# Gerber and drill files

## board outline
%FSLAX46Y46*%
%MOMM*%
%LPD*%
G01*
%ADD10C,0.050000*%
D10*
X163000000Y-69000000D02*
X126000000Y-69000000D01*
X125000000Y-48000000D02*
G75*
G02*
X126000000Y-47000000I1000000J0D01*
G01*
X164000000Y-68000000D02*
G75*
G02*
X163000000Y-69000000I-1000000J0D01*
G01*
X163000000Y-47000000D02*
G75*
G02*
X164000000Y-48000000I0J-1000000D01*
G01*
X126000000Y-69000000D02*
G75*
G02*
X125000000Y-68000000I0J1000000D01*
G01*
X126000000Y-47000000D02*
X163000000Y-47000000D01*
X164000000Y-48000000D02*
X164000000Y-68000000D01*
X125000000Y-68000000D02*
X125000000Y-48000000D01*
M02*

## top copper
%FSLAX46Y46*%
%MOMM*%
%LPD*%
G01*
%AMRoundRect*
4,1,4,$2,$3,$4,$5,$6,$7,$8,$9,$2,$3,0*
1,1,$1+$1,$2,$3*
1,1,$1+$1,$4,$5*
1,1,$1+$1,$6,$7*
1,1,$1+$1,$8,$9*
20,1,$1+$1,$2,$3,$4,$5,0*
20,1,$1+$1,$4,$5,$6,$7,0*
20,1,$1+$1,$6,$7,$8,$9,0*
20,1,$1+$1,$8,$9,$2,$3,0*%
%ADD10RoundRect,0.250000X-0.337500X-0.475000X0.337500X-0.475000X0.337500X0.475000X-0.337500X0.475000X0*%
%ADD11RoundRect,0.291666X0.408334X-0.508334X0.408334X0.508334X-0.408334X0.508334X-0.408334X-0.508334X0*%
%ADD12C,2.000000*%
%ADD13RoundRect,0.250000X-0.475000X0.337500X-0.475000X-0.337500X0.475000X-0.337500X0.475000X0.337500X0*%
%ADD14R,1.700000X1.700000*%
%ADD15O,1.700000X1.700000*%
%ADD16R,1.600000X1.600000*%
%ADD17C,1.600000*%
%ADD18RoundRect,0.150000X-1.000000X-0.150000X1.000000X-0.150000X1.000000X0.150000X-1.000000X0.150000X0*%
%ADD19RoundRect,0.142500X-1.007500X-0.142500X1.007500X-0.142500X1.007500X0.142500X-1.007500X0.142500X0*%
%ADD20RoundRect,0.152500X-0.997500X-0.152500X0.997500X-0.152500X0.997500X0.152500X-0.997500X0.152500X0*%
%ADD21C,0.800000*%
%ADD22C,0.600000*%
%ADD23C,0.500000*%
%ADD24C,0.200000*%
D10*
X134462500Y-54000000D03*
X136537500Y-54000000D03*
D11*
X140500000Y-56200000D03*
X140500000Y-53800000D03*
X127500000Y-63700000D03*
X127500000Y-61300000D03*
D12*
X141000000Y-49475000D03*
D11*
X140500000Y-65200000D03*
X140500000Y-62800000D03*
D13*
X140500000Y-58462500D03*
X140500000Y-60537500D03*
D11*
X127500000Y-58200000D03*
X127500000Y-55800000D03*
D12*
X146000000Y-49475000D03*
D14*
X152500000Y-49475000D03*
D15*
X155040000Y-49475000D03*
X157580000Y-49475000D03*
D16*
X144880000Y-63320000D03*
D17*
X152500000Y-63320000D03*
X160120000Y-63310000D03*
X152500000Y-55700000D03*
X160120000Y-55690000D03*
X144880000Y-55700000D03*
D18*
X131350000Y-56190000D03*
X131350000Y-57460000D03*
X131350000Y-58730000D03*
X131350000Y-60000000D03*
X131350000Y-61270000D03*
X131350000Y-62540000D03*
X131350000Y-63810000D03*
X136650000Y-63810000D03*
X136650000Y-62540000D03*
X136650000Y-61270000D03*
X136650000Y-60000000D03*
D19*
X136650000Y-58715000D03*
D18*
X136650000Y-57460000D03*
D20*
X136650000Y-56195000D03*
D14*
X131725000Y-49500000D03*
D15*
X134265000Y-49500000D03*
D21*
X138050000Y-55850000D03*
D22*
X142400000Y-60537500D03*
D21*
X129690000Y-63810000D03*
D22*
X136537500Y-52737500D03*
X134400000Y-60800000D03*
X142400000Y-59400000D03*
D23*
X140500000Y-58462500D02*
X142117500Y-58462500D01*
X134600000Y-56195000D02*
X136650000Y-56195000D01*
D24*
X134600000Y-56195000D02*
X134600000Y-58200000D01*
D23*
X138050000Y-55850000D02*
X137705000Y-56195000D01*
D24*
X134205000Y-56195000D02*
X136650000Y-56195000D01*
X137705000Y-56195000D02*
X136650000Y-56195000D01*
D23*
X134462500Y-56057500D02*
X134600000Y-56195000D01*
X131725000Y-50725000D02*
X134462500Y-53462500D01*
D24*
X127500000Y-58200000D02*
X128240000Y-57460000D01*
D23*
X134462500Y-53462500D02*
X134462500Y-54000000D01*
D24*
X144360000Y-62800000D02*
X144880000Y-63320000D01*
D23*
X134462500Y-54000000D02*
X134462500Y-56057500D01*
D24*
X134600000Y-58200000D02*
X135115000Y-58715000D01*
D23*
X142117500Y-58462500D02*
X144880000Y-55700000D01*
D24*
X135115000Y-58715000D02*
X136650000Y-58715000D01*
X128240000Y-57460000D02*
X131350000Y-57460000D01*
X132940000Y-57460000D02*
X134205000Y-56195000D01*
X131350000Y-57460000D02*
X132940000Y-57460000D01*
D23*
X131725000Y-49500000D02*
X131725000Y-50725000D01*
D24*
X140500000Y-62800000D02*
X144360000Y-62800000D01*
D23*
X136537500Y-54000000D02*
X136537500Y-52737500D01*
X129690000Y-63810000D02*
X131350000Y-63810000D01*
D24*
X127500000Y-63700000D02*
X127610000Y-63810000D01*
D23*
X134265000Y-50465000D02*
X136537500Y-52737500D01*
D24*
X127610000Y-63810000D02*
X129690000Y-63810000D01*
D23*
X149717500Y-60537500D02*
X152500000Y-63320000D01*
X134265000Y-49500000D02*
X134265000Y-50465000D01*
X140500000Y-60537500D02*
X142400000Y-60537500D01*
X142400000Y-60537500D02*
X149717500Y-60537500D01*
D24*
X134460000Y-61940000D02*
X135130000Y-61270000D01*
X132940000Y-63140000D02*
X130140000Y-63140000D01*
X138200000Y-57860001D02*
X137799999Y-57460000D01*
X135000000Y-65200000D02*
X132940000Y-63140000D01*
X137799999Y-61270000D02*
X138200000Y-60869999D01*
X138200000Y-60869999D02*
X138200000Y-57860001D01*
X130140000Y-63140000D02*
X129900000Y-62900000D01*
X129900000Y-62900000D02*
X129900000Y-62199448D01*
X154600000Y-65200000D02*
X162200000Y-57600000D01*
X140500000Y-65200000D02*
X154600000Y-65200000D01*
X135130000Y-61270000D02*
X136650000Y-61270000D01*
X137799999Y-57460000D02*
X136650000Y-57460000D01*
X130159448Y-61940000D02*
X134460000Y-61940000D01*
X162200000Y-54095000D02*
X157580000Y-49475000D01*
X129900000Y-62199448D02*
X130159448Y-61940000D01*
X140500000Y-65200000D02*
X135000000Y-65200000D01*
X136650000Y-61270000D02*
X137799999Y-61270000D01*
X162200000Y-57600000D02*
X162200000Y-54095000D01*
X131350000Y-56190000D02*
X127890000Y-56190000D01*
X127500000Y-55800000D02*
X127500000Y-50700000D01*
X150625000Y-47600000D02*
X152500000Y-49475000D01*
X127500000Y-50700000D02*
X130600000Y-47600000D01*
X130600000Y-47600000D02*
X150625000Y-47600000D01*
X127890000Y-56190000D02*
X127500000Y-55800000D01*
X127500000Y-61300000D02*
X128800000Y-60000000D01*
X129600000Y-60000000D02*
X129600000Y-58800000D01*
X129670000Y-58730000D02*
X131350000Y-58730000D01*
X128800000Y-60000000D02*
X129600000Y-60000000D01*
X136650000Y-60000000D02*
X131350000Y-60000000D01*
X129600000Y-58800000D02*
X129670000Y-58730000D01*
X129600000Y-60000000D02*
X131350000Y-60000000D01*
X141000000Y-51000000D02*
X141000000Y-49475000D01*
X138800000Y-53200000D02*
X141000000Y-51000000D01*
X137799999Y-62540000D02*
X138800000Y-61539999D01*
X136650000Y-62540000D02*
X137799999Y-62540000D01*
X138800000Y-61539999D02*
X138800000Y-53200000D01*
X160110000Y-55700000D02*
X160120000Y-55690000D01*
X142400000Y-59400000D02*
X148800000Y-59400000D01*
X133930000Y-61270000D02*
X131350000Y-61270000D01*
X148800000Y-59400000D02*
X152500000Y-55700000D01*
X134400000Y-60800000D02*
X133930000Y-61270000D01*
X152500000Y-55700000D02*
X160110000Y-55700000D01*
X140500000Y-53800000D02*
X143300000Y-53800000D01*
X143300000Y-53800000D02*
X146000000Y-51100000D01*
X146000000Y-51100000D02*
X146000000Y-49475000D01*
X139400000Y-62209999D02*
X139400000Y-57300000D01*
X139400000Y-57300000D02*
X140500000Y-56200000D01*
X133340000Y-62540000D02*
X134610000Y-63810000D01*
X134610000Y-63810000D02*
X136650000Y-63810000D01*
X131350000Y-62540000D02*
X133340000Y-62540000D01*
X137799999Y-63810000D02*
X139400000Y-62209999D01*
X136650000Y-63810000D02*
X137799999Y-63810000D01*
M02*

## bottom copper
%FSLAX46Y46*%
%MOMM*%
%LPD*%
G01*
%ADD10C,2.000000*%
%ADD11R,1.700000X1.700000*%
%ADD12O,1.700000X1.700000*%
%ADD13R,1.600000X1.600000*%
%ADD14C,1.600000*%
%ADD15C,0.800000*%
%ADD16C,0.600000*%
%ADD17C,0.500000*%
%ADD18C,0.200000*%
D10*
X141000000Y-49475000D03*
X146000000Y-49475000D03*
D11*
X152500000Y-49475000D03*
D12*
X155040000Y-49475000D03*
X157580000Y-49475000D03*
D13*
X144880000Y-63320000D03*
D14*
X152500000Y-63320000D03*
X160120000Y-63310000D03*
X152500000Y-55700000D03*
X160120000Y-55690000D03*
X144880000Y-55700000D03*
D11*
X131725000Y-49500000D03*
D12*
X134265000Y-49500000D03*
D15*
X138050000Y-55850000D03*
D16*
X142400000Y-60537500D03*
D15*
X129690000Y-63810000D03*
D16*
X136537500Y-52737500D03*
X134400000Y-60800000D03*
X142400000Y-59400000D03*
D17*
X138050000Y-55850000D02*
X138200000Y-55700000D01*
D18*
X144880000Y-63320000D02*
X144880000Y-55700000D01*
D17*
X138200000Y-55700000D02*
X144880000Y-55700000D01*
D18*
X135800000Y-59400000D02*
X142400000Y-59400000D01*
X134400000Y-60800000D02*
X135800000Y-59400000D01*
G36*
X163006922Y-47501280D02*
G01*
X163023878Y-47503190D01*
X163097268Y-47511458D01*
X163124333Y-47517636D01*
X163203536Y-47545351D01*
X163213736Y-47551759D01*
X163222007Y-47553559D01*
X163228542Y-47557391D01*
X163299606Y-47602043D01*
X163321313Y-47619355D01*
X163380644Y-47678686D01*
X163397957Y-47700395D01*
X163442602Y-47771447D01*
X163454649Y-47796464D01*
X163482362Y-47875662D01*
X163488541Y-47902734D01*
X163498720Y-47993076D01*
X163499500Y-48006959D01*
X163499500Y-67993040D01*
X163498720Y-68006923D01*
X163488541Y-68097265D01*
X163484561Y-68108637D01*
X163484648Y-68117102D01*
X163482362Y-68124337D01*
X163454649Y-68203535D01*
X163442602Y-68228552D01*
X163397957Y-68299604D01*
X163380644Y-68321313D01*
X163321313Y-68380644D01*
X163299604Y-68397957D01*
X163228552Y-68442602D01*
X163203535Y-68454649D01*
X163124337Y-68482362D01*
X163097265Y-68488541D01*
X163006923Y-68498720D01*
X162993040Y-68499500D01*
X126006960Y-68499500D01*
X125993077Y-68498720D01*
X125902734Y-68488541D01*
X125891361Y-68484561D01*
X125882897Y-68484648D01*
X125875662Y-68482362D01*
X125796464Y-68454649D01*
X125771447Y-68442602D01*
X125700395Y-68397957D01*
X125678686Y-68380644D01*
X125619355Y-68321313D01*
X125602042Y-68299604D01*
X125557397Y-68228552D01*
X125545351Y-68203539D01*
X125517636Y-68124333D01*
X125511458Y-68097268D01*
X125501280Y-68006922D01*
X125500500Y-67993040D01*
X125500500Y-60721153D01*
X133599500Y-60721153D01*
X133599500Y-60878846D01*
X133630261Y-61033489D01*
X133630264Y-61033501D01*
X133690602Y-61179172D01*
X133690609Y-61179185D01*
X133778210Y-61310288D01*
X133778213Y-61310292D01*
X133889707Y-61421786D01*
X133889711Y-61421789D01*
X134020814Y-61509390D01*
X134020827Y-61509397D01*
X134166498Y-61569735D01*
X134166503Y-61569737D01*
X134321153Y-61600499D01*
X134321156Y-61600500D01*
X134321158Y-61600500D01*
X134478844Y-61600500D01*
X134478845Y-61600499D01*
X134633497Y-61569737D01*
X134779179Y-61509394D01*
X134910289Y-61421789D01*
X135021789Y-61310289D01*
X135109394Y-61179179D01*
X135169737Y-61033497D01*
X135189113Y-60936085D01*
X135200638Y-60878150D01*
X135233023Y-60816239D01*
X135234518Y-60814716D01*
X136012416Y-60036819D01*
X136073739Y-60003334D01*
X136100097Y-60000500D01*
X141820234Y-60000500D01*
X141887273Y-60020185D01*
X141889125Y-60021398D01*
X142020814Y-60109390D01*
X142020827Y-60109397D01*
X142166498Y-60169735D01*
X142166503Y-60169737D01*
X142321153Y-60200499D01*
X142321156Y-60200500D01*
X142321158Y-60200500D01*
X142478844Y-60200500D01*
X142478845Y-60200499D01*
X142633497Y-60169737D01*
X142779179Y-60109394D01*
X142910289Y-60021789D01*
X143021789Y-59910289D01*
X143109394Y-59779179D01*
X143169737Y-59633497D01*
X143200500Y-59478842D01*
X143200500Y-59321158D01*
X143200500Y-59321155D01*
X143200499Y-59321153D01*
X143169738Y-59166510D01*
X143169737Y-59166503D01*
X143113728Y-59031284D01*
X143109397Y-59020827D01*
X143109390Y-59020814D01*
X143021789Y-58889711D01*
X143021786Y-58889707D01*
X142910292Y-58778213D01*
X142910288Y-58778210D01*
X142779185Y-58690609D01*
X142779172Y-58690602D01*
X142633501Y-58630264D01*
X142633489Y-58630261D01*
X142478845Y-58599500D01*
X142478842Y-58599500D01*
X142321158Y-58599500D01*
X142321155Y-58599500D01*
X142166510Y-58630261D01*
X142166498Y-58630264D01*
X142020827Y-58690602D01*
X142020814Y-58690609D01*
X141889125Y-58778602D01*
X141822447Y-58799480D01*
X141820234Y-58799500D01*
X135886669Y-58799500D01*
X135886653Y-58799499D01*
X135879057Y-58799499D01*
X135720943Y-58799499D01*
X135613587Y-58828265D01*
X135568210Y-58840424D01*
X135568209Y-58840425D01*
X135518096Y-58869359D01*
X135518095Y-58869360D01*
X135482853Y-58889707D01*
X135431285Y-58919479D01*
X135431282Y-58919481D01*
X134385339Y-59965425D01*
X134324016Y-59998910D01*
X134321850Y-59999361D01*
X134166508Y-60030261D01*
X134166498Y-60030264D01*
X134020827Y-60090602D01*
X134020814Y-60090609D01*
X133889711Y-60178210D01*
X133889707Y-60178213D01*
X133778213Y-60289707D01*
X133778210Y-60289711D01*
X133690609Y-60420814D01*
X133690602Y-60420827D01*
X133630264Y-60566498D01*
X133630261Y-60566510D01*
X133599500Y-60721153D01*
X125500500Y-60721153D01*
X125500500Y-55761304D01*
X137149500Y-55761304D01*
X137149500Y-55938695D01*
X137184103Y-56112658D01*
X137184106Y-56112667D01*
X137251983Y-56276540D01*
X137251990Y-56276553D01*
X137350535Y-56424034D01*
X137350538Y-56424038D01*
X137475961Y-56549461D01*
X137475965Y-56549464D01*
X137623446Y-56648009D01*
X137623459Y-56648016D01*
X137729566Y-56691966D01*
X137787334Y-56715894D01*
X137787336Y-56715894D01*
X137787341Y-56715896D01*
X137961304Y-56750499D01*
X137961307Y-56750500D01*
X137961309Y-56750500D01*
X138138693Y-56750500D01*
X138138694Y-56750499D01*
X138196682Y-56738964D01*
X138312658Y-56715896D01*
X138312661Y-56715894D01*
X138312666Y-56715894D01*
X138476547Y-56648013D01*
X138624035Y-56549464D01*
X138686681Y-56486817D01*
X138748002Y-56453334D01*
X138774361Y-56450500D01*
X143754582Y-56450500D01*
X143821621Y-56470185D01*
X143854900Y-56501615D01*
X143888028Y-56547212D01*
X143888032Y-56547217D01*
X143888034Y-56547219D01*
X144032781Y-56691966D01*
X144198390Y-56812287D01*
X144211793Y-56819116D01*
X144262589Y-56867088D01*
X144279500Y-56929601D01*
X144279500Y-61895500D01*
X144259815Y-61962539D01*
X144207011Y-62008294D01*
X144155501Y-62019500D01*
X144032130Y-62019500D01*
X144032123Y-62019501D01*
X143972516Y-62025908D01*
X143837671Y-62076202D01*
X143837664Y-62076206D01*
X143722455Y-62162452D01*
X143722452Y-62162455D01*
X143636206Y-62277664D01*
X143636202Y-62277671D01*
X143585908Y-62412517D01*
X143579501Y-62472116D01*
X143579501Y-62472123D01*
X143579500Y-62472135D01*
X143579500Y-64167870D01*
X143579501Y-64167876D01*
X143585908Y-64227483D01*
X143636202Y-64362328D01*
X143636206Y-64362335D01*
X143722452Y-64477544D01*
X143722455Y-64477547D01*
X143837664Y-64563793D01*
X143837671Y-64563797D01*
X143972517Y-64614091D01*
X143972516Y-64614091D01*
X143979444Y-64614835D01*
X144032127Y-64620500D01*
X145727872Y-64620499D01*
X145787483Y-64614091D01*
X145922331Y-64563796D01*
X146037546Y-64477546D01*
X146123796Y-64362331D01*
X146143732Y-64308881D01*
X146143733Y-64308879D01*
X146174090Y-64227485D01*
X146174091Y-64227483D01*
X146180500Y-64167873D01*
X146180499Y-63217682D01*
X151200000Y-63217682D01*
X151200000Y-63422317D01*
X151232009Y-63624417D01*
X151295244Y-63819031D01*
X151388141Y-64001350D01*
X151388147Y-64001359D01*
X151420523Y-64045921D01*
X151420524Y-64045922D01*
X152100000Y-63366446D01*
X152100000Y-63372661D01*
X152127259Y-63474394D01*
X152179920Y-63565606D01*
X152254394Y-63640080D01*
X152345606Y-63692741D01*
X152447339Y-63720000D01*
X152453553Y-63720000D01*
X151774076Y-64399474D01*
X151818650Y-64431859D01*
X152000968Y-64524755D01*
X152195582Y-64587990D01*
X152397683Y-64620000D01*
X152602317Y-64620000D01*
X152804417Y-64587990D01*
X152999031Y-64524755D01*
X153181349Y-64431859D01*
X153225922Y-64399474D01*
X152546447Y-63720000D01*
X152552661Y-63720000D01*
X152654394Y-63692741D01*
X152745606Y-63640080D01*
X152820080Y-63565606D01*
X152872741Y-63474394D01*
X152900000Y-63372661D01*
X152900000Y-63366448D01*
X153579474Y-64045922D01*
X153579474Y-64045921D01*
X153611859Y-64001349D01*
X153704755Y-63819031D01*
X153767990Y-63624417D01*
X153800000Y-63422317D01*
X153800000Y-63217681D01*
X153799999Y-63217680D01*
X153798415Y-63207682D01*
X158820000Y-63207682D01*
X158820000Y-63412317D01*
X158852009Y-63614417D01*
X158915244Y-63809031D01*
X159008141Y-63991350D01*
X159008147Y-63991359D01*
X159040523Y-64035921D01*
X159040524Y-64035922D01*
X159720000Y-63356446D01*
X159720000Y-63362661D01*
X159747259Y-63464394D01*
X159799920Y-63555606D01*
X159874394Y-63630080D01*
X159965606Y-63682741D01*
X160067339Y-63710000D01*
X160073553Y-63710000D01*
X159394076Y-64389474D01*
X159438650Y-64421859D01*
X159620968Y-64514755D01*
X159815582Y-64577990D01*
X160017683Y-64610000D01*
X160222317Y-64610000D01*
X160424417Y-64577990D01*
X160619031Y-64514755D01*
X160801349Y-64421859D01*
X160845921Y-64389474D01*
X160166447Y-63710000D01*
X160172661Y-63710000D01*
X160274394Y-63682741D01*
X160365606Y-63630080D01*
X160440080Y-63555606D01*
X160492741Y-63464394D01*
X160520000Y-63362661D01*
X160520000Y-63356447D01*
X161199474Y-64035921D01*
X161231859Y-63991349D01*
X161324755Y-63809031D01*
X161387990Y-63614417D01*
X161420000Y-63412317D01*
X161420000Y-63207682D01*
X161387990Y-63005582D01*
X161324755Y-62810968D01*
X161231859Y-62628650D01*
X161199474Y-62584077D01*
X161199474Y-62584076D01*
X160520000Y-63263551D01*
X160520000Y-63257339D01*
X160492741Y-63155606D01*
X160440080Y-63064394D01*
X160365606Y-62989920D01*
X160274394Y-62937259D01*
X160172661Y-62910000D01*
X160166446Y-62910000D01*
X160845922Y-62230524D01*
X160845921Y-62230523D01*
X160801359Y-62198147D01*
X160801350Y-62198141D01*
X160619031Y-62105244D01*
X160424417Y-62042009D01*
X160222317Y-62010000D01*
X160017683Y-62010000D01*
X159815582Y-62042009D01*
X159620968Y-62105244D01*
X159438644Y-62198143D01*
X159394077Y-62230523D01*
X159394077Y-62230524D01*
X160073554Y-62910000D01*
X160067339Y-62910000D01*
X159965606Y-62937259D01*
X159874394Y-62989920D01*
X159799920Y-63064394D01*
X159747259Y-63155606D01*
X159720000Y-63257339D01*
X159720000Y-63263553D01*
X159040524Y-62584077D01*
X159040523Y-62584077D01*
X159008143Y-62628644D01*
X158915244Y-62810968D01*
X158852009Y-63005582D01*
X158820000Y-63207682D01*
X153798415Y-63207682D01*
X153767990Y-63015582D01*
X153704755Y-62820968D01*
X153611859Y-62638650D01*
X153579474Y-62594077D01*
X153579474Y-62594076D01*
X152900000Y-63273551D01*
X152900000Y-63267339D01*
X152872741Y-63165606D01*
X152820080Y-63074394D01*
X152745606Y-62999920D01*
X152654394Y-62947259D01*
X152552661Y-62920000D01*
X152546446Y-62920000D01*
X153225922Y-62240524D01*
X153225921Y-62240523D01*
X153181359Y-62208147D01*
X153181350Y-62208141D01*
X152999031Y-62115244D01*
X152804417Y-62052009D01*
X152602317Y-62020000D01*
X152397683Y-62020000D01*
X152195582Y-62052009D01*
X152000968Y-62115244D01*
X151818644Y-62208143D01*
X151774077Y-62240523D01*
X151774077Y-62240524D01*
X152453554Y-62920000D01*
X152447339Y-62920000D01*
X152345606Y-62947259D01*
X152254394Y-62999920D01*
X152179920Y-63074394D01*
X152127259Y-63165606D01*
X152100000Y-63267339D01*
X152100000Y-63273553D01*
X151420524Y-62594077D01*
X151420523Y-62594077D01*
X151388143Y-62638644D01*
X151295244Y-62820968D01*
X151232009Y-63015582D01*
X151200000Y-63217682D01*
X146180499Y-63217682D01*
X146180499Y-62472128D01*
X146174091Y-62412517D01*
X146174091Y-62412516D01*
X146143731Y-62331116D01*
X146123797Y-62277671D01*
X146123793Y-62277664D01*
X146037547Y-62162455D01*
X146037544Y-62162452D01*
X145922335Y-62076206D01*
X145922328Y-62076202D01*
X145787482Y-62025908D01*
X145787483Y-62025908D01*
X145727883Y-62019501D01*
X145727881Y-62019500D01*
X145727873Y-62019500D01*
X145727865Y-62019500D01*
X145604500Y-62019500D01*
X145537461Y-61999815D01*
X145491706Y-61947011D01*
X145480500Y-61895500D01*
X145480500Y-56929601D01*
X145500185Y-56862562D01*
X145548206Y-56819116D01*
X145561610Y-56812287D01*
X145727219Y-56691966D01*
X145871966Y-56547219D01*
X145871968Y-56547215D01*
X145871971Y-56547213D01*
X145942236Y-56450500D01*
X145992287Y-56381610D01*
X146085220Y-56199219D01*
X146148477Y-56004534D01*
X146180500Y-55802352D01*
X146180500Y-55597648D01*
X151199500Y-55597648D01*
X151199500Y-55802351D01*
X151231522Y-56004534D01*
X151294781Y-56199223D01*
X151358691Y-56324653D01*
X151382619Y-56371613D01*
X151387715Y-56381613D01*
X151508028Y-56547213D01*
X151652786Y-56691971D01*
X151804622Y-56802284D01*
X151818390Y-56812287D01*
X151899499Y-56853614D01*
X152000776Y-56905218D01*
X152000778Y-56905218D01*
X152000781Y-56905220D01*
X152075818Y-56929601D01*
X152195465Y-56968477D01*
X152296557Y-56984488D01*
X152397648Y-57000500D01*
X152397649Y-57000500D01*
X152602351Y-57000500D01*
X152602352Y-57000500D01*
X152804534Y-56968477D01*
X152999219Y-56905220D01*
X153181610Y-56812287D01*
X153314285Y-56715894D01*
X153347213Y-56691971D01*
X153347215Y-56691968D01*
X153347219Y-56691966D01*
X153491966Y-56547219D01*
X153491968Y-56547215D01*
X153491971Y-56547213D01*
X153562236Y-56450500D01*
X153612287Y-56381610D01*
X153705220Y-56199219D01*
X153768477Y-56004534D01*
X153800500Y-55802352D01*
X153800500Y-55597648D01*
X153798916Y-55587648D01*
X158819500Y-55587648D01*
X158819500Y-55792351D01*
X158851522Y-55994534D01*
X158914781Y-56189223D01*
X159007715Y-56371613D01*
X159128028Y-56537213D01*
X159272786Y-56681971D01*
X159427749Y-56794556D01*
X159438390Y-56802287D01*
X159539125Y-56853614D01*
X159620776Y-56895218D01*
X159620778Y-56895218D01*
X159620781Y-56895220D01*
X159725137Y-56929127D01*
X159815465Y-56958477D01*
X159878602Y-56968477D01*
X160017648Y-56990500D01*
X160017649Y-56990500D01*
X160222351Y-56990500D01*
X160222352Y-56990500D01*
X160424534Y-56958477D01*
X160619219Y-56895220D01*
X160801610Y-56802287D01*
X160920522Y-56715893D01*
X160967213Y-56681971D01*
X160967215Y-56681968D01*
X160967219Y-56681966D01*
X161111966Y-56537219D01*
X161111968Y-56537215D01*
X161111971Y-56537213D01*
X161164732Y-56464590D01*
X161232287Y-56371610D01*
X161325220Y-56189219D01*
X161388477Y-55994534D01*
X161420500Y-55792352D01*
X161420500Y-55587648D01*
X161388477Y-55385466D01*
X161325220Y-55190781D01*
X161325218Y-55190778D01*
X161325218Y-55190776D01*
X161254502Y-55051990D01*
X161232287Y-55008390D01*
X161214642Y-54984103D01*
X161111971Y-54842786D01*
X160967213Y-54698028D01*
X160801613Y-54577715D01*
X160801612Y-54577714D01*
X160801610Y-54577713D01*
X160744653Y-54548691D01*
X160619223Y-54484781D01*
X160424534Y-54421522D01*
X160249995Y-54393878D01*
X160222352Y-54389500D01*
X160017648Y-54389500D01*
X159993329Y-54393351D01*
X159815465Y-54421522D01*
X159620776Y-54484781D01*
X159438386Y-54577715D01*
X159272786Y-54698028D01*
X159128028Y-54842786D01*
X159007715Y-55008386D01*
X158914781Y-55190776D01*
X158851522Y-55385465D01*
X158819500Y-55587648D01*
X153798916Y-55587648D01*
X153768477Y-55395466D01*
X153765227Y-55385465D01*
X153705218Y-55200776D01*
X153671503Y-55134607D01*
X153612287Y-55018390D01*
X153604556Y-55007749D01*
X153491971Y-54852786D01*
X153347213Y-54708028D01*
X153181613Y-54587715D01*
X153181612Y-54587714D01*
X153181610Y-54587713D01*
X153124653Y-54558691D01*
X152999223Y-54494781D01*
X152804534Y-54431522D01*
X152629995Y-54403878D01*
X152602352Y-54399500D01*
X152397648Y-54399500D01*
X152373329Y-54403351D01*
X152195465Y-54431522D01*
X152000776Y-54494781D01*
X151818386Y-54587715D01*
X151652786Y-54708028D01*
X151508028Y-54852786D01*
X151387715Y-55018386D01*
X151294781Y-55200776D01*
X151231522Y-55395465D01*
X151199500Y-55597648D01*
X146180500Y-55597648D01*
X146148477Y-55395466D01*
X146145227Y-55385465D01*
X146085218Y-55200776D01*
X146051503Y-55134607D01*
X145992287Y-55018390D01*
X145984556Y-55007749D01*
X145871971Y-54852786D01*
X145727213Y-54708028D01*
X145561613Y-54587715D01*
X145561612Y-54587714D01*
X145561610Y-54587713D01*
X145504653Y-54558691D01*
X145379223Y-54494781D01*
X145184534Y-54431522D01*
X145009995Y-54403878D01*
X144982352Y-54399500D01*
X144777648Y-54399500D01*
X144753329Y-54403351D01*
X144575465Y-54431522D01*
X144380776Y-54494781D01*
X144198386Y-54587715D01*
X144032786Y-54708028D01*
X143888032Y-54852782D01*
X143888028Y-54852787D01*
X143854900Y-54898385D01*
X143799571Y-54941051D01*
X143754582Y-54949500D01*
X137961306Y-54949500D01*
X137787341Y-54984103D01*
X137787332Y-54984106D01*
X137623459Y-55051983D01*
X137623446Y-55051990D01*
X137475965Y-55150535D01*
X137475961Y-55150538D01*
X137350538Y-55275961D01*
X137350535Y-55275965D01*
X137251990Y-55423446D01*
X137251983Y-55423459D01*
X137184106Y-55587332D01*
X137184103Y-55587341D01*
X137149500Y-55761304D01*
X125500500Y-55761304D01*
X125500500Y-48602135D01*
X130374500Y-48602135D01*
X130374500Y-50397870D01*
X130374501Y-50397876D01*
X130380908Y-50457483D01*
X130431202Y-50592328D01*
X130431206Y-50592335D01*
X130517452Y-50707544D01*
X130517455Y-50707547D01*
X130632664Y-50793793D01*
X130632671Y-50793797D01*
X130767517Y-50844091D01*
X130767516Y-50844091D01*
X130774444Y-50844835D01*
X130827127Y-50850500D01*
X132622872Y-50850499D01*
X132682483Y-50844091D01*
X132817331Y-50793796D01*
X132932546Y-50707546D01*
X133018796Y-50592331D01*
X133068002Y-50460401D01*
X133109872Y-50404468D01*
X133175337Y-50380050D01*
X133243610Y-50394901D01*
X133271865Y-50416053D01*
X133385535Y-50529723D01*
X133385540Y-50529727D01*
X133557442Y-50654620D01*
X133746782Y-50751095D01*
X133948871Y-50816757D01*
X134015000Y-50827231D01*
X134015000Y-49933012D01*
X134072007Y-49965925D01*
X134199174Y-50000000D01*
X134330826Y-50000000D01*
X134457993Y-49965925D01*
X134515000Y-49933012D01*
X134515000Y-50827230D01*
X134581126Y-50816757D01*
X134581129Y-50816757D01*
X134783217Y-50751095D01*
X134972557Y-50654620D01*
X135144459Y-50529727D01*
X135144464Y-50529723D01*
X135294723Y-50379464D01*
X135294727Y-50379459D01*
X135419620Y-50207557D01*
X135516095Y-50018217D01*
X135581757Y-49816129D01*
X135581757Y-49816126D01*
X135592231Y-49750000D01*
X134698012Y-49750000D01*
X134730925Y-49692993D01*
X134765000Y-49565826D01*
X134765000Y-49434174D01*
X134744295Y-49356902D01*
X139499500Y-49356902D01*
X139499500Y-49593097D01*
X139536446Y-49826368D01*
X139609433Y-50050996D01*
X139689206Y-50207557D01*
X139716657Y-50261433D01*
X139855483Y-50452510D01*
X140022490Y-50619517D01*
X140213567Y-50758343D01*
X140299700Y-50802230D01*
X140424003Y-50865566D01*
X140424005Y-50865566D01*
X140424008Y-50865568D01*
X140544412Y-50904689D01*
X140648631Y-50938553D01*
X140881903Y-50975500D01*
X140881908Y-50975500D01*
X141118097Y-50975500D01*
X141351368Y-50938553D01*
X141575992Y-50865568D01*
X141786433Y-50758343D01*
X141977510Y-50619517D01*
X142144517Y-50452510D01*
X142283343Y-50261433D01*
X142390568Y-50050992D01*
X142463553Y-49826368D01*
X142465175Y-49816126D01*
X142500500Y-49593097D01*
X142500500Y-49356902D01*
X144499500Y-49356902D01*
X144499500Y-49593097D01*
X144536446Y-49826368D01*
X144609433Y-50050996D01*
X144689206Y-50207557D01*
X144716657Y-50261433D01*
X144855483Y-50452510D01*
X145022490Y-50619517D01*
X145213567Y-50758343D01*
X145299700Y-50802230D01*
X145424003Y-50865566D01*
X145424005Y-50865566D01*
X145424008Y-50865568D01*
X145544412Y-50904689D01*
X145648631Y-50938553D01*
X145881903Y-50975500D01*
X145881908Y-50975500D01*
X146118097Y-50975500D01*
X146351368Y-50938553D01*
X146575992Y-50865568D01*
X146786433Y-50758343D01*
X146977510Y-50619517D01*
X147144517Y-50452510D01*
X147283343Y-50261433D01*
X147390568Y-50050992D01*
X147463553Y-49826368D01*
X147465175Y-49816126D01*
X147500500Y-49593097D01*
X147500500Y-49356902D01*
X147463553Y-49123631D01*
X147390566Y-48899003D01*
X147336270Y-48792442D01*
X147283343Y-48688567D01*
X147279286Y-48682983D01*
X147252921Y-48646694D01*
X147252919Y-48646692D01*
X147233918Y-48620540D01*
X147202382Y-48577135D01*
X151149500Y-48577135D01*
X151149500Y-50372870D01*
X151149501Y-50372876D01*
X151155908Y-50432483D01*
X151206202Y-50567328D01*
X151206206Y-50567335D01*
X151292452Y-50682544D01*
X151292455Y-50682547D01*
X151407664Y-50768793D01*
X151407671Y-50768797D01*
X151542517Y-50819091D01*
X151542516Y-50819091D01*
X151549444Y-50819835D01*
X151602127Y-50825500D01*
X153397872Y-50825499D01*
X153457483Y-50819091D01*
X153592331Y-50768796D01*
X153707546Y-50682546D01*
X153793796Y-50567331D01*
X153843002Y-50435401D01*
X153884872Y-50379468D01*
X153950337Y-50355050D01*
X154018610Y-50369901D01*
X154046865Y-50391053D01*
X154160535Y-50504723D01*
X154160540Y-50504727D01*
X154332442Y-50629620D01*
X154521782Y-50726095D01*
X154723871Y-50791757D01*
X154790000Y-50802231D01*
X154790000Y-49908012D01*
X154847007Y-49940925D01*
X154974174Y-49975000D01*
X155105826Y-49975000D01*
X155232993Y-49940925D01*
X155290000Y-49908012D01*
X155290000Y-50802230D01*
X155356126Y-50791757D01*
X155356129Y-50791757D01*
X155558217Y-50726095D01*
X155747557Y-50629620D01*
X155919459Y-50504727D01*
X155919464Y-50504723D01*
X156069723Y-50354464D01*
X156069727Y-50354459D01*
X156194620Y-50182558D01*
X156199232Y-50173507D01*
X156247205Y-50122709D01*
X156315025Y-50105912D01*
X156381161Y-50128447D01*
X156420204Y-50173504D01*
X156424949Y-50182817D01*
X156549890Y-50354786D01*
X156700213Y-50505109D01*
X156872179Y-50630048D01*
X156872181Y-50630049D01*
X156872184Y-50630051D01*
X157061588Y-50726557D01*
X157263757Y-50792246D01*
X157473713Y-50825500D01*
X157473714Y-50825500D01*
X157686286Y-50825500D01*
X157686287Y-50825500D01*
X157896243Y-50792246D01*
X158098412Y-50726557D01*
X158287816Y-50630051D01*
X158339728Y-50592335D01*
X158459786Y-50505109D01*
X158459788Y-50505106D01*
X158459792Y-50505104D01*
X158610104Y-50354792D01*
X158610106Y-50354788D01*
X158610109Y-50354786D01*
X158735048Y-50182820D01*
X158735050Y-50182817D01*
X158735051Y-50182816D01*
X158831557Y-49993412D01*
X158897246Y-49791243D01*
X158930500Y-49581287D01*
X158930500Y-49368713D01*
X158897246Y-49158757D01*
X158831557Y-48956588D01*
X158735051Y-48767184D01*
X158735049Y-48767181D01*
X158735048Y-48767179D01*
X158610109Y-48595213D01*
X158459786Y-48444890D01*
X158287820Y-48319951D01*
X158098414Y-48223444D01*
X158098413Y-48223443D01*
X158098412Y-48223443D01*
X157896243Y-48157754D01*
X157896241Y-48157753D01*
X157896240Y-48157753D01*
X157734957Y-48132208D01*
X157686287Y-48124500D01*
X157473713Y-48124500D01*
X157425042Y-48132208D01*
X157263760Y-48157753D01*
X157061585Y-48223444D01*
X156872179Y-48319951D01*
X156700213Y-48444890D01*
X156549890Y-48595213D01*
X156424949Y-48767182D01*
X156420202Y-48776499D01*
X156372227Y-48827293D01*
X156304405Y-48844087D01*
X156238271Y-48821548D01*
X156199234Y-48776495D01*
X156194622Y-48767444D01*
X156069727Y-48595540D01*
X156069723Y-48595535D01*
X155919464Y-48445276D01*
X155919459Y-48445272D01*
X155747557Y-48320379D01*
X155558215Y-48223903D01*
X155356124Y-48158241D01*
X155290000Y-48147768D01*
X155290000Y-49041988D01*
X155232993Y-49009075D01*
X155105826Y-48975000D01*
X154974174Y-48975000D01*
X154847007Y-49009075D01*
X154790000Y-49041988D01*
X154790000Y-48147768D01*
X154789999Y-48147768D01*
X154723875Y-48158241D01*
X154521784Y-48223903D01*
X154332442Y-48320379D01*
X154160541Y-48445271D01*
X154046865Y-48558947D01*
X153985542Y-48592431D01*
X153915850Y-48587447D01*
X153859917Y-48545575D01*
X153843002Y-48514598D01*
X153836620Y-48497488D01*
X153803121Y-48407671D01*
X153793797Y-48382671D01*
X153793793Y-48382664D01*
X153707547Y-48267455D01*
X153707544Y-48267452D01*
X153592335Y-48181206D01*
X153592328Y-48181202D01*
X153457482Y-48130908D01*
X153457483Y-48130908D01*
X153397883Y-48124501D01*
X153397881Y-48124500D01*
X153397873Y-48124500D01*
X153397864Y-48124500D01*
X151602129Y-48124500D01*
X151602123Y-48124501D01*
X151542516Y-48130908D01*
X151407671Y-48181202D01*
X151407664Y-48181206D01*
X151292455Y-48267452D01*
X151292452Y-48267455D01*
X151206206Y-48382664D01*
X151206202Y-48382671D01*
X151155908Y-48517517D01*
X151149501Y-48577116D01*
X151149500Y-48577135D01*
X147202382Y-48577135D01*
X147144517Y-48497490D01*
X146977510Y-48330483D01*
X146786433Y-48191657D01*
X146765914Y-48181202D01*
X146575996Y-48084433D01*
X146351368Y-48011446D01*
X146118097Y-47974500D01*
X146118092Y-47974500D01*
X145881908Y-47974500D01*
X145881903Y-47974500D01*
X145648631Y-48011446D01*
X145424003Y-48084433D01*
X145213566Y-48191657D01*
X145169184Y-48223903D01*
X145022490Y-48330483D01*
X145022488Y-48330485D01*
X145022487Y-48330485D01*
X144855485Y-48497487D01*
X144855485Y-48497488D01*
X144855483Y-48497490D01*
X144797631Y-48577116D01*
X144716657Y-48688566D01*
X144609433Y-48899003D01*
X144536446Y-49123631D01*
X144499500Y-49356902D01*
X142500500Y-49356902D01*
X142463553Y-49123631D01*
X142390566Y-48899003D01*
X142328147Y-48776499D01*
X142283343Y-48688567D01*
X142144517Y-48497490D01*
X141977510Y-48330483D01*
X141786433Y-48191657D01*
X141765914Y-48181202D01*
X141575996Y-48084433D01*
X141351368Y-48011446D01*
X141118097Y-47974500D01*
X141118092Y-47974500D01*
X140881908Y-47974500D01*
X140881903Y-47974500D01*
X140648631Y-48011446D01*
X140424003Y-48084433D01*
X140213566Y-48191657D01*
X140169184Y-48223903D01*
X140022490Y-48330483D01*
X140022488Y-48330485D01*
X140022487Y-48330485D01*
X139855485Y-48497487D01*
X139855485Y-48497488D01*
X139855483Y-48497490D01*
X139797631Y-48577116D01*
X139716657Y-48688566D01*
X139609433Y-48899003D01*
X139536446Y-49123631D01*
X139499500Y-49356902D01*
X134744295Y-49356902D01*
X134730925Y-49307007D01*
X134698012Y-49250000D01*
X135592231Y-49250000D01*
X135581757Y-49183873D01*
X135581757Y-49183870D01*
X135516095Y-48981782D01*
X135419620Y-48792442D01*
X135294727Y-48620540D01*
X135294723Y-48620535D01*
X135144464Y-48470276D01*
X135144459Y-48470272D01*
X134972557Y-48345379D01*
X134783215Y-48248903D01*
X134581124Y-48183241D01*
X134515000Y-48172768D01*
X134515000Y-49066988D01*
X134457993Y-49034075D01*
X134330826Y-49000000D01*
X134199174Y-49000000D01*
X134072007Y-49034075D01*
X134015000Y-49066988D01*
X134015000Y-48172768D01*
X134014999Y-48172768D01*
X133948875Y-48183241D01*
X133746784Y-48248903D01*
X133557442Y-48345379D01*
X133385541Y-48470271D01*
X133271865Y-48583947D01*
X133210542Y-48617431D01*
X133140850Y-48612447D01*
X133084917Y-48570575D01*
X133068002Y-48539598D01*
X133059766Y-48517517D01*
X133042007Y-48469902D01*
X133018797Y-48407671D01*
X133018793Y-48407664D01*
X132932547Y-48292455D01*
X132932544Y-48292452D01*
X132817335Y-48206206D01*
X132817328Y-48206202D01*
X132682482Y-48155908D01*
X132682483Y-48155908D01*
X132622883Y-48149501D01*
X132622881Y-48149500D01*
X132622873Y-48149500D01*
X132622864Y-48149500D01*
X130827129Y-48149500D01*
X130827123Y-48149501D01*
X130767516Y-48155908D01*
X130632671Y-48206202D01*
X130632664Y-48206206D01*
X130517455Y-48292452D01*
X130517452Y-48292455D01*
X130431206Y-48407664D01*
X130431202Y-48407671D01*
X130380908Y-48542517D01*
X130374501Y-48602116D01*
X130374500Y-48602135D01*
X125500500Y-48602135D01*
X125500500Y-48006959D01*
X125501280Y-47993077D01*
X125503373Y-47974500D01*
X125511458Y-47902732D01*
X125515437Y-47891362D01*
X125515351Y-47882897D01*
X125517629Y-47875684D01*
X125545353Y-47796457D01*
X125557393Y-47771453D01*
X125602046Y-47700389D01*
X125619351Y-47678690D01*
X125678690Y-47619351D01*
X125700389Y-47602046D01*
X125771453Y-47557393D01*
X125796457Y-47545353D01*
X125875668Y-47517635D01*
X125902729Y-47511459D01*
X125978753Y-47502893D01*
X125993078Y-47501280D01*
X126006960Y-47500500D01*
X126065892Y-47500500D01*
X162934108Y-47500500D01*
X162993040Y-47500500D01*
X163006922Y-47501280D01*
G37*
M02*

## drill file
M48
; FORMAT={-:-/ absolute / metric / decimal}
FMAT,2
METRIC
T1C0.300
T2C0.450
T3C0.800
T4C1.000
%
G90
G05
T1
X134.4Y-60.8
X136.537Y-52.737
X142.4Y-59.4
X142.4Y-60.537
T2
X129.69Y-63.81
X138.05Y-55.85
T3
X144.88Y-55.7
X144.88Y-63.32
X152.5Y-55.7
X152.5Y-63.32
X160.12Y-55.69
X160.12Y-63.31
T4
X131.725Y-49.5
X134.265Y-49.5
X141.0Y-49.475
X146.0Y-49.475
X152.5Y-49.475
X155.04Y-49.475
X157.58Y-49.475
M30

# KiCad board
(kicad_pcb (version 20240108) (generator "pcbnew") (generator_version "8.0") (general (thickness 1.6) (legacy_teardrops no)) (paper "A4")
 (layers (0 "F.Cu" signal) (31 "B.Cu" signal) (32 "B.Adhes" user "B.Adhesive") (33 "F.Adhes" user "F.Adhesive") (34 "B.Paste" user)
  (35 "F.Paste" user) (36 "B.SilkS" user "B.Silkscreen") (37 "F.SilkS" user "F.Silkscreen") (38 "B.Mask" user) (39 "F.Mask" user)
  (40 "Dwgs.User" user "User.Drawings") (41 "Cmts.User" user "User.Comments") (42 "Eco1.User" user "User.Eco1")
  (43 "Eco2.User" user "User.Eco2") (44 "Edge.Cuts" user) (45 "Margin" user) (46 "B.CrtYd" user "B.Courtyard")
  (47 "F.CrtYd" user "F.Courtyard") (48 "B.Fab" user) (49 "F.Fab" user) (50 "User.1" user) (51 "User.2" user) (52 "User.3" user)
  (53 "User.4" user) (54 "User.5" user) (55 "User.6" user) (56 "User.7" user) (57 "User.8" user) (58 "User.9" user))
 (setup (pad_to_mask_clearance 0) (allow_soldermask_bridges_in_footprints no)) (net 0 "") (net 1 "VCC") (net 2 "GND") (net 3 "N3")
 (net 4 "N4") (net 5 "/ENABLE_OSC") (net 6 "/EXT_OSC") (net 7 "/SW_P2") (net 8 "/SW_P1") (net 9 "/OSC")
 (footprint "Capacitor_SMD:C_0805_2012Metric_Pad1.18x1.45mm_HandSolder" (layer "F.Cu") (at 135.5 54)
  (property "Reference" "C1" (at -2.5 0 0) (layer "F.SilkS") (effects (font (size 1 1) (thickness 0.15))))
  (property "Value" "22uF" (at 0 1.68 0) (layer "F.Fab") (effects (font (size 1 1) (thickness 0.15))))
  (pad "1" smd roundrect (at -1.0375 0) (size 1.175 1.45) (layers "F.Cu" "F.Paste" "F.Mask") (roundrect_rratio 0.212766) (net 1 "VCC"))
  (pad "2" smd roundrect (at 1.0375 0) (size 1.175 1.45) (layers "F.Cu" "F.Paste" "F.Mask") (roundrect_rratio 0.212766) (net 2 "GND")))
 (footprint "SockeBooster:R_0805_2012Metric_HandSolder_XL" (layer "F.Cu") (at 140.5 55 90)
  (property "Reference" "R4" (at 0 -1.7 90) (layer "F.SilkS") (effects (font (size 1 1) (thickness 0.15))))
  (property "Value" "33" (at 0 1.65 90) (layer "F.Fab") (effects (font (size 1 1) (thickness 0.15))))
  (pad "1" smd roundrect (at -1.2 0 90) (size 1.6 1.4) (layers "F.Cu" "F.Paste" "F.Mask") (roundrect_rratio 0.208333) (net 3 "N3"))
  (pad "2" smd roundrect (at 1.2 0 90) (size 1.6 1.4) (layers "F.Cu" "F.Paste" "F.Mask") (roundrect_rratio 0.208333) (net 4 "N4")))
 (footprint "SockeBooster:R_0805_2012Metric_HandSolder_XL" (layer "F.Cu") (at 127.5 62.5 90)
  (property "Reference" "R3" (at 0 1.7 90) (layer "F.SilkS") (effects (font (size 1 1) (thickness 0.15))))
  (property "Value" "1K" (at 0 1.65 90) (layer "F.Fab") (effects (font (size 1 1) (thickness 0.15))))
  (pad "1" smd roundrect (at -1.2 0 90) (size 1.6 1.4) (layers "F.Cu" "F.Paste" "F.Mask") (roundrect_rratio 0.208333) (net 2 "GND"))
  (pad "2" smd roundrect (at 1.2 0 90) (size 1.6 1.4) (layers "F.Cu" "F.Paste" "F.Mask") (roundrect_rratio 0.208333) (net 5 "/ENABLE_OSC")))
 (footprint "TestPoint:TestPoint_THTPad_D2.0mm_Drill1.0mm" (layer "F.Cu") (at 141 49.475)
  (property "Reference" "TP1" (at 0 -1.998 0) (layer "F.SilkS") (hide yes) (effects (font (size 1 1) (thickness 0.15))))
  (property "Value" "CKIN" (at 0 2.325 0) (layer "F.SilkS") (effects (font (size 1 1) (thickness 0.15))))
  (pad "1" thru_hole circle (at 0 0) (size 2 2) (drill 1) (layers "*.Cu" "*.Mask") (remove_unused_layers no) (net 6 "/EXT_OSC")))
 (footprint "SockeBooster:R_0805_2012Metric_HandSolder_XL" (layer "F.Cu") (at 140.5 64 90)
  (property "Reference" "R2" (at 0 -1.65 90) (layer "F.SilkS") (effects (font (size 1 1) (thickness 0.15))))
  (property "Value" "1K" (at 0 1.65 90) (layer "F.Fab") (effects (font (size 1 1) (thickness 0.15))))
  (pad "1" smd roundrect (at -1.2 0 90) (size 1.6 1.4) (layers "F.Cu" "F.Paste" "F.Mask") (roundrect_rratio 0.208333) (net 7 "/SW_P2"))
  (pad "2" smd roundrect (at 1.2 0 90) (size 1.6 1.4) (layers "F.Cu" "F.Paste" "F.Mask") (roundrect_rratio 0.208333) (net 1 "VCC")))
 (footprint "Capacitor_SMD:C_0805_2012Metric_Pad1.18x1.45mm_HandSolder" (layer "F.Cu") (at 140.5 59.5 -90)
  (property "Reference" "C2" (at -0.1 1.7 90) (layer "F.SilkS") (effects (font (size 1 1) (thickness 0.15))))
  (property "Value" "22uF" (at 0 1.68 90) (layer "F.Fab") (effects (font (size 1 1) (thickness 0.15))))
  (pad "1" smd roundrect (at -1.0375 0 270) (size 1.175 1.45) (layers "F.Cu" "F.Paste" "F.Mask") (roundrect_rratio 0.212766) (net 1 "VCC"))
  (pad "2" smd roundrect (at 1.0375 0 270) (size 1.175 1.45) (layers "F.Cu" "F.Paste" "F.Mask") (roundrect_rratio 0.212766) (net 2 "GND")))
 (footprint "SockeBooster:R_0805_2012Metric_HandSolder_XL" (layer "F.Cu") (at 127.5 57 90)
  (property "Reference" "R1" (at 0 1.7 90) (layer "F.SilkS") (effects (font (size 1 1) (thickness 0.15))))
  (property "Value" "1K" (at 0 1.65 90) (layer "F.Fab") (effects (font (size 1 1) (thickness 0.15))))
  (pad "1" smd roundrect (at -1.2 0 90) (size 1.6 1.4) (layers "F.Cu" "F.Paste" "F.Mask") (roundrect_rratio 0.208333) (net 1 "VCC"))
  (pad "2" smd roundrect (at 1.2 0 90) (size 1.6 1.4) (layers "F.Cu" "F.Paste" "F.Mask") (roundrect_rratio 0.208333) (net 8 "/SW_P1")))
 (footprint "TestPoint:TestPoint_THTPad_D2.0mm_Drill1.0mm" (layer "F.Cu") (at 146 49.475)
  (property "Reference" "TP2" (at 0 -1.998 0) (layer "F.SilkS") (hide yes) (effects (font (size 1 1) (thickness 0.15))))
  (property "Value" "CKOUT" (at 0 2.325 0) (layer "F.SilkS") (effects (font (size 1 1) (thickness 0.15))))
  (pad "1" thru_hole circle (at 0 0) (size 2 2) (drill 1) (layers "*.Cu" "*.Mask") (remove_unused_layers no) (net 4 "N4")))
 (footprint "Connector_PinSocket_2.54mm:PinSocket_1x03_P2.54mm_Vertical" (layer "F.Cu") (at 152.5 49.475 90)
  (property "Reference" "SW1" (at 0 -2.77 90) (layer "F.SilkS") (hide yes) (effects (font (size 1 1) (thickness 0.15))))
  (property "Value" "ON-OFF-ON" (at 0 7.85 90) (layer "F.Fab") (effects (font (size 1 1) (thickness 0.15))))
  (pad "1" thru_hole rect (at 0 0 90) (size 1.7 1.7) (drill 1) (layers "*.Cu" "*.Mask") (remove_unused_layers no) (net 8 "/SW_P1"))
  (pad "2" thru_hole oval (at 0 2.54 90) (size 1.7 1.7) (drill 1) (layers "*.Cu" "*.Mask") (remove_unused_layers no) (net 2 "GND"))
  (pad "3" thru_hole oval (at 0 5.08 90) (size 1.7 1.7) (drill 1) (layers "*.Cu" "*.Mask") (remove_unused_layers no) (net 7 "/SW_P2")))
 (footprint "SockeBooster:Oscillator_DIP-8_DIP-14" (layer "F.Cu") (at 144.88 63.32)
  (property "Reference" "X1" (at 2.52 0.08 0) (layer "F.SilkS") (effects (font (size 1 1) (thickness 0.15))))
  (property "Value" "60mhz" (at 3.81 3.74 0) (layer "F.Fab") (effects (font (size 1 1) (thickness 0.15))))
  (pad "1" thru_hole rect (at 0 0) (size 1.6 1.6) (drill 0.8) (layers "*.Cu" "*.Mask") (remove_unused_layers no) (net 1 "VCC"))
  (pad "4" thru_hole circle (at 7.62 0) (size 1.6 1.6) (drill 0.8) (layers "*.Cu" "*.Mask") (remove_unused_layers no) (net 2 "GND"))
  (pad "4" thru_hole circle (at 15.24 -0.01) (size 1.6 1.6) (drill 0.8) (layers "*.Cu" "*.Mask") (remove_unused_layers no) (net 2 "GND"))
  (pad "5" thru_hole circle (at 7.62 -7.62) (size 1.6 1.6) (drill 0.8) (layers "*.Cu" "*.Mask") (remove_unused_layers no) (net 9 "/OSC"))
  (pad "5" thru_hole circle (at 15.24 -7.63) (size 1.6 1.6) (drill 0.8) (layers "*.Cu" "*.Mask") (remove_unused_layers no) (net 9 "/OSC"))
  (pad "8" thru_hole circle (at 0 -7.62) (size 1.6 1.6) (drill 0.8) (layers "*.Cu" "*.Mask") (remove_unused_layers no) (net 1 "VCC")))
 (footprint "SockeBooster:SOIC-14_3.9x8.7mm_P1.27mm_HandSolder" (layer "F.Cu") (at 134 60)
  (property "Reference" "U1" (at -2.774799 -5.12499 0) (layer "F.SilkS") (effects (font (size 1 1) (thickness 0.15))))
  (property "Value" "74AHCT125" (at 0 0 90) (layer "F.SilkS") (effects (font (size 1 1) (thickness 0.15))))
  (pad "1" smd roundrect (at -2.65 -3.81) (size 2.3 0.6) (layers "F.Cu" "F.Paste" "F.Mask") (roundrect_rratio 0.25) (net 8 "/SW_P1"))
  (pad "2" smd roundrect (at -2.65 -2.54) (size 2.3 0.6) (layers "F.Cu" "F.Paste" "F.Mask") (roundrect_rratio 0.25) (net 1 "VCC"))
  (pad "3" smd roundrect (at -2.65 -1.27) (size 2.3 0.6) (layers "F.Cu" "F.Paste" "F.Mask") (roundrect_rratio 0.25) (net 5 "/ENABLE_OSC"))
  (pad "4" smd roundrect (at -2.65 0) (size 2.3 0.6) (layers "F.Cu" "F.Paste" "F.Mask") (roundrect_rratio 0.25) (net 5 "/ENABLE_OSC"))
  (pad "5" smd roundrect (at -2.65 1.27) (size 2.3 0.6) (layers "F.Cu" "F.Paste" "F.Mask") (roundrect_rratio 0.25) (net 9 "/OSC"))
  (pad "6" smd roundrect (at -2.65 2.54) (size 2.3 0.6) (layers "F.Cu" "F.Paste" "F.Mask") (roundrect_rratio 0.25) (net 3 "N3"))
  (pad "7" smd roundrect (at -2.65 3.81) (size 2.3 0.6) (layers "F.Cu" "F.Paste" "F.Mask") (roundrect_rratio 0.25) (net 2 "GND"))
  (pad "8" smd roundrect (at 2.65 3.81) (size 2.3 0.6) (layers "F.Cu" "F.Paste" "F.Mask") (roundrect_rratio 0.25) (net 3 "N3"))
  (pad "9" smd roundrect (at 2.65 2.54) (size 2.3 0.6) (layers "F.Cu" "F.Paste" "F.Mask") (roundrect_rratio 0.25) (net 6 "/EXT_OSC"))
  (pad "10" smd roundrect (at 2.65 1.27) (size 2.3 0.6) (layers "F.Cu" "F.Paste" "F.Mask") (roundrect_rratio 0.25) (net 7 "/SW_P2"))
  (pad "11" smd roundrect (at 2.65 0) (size 2.3 0.6) (layers "F.Cu" "F.Paste" "F.Mask") (roundrect_rratio 0.25) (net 5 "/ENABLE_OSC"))
  (pad "12" smd roundrect (at 2.65 -1.285) (size 2.3 0.57) (layers "F.Cu" "F.Paste" "F.Mask") (roundrect_rratio 0.25) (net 1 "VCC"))
  (pad "13" smd roundrect (at 2.65 -2.54) (size 2.3 0.6) (layers "F.Cu" "F.Paste" "F.Mask") (roundrect_rratio 0.25) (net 7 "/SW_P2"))
  (pad "14" smd roundrect (at 2.65 -3.805) (size 2.3 0.61) (layers "F.Cu" "F.Paste" "F.Mask") (roundrect_rratio 0.25) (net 1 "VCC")))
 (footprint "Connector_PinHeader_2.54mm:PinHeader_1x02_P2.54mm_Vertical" (layer "F.Cu") (at 131.725 49.5 90)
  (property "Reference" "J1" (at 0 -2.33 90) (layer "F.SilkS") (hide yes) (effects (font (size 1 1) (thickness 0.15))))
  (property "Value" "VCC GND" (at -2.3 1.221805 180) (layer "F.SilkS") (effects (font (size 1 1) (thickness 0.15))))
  (pad "1" thru_hole rect (at 0 0 90) (size 1.7 1.7) (drill 1) (layers "*.Cu" "*.Mask") (remove_unused_layers no) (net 1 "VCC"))
  (pad "2" thru_hole oval (at 0 2.54 90) (size 1.7 1.7) (drill 1) (layers "*.Cu" "*.Mask") (remove_unused_layers no) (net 2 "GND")))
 (gr_line (start 163 69) (end 126 69) (stroke (width 0.05) (type default)) (layer "Edge.Cuts"))
 (gr_arc (start 125 48) (mid 125.292893 47.292893) (end 126 47) (stroke (width 0.05) (type default)) (layer "Edge.Cuts"))
 (gr_arc (start 164 68) (mid 163.707107 68.707107) (end 163 69) (stroke (width 0.05) (type default)) (layer "Edge.Cuts"))
 (gr_arc (start 163 47) (mid 163.707107 47.292893) (end 164 48) (stroke (width 0.05) (type default)) (layer "Edge.Cuts"))
 (gr_arc (start 126 69) (mid 125.292893 68.707107) (end 125 68) (stroke (width 0.05) (type default)) (layer "Edge.Cuts"))
 (gr_line (start 126 47) (end 163 47) (stroke (width 0.05) (type default)) (layer "Edge.Cuts"))
 (gr_line (start 164 48) (end 164 68) (stroke (width 0.05) (type default)) (layer "Edge.Cuts"))
 (gr_line (start 125 68) (end 125 48) (stroke (width 0.05) (type default)) (layer "Edge.Cuts"))
 (segment (start 140.5 58.4625) (end 142.1175 58.4625) (width 0.5) (layer "F.Cu") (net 1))
 (segment (start 134.6 56.195) (end 136.65 56.195) (width 0.5) (layer "F.Cu") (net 1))
 (segment (start 134.6 56.195) (end 134.6 58.2) (width 0.2) (layer "F.Cu") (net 1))
 (segment (start 138.05 55.85) (end 137.705 56.195) (width 0.5) (layer "F.Cu") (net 1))
 (segment (start 134.205 56.195) (end 136.65 56.195) (width 0.2) (layer "F.Cu") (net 1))
 (segment (start 137.705 56.195) (end 136.65 56.195) (width 0.2) (layer "F.Cu") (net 1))
 (segment (start 134.4625 56.0575) (end 134.6 56.195) (width 0.5) (layer "F.Cu") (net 1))
 (segment (start 131.725 50.725) (end 134.4625 53.4625) (width 0.5) (layer "F.Cu") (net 1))
 (segment (start 127.5 58.2) (end 128.24 57.46) (width 0.2) (layer "F.Cu") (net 1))
 (segment (start 134.4625 53.4625) (end 134.4625 54) (width 0.5) (layer "F.Cu") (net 1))
 (segment (start 144.36 62.8) (end 144.88 63.32) (width 0.2) (layer "F.Cu") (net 1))
 (segment (start 134.4625 54) (end 134.4625 56.0575) (width 0.5) (layer "F.Cu") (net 1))
 (segment (start 134.6 58.2) (end 135.115 58.715) (width 0.2) (layer "F.Cu") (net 1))
 (segment (start 142.1175 58.4625) (end 144.88 55.7) (width 0.5) (layer "F.Cu") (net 1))
 (segment (start 135.115 58.715) (end 136.65 58.715) (width 0.2) (layer "F.Cu") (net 1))
 (segment (start 128.24 57.46) (end 131.35 57.46) (width 0.2) (layer "F.Cu") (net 1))
 (segment (start 132.94 57.46) (end 134.205 56.195) (width 0.2) (layer "F.Cu") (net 1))
 (segment (start 131.35 57.46) (end 132.94 57.46) (width 0.2) (layer "F.Cu") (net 1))
 (segment (start 131.725 49.5) (end 131.725 50.725) (width 0.5) (layer "F.Cu") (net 1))
 (segment (start 140.5 62.8) (end 144.36 62.8) (width 0.2) (layer "F.Cu") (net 1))
 (via (at 138.05 55.85) (size 0.8) (drill 0.45) (layers "F.Cu" "B.Cu") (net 1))
 (segment (start 138.05 55.85) (end 138.2 55.7) (width 0.5) (layer "B.Cu") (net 1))
 (segment (start 144.88 63.32) (end 144.88 55.7) (width 0.2) (layer "B.Cu") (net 1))
 (segment (start 138.2 55.7) (end 144.88 55.7) (width 0.5) (layer "B.Cu") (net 1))
 (segment (start 136.5375 54) (end 136.5375 52.7375) (width 0.5) (layer "F.Cu") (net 2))
 (segment (start 129.69 63.81) (end 131.35 63.81) (width 0.5) (layer "F.Cu") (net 2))
 (segment (start 127.5 63.7) (end 127.61 63.81) (width 0.2) (layer "F.Cu") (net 2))
 (segment (start 134.265 50.465) (end 136.5375 52.7375) (width 0.5) (layer "F.Cu") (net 2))
 (segment (start 127.61 63.81) (end 129.69 63.81) (width 0.2) (layer "F.Cu") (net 2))
 (segment (start 149.7175 60.5375) (end 152.5 63.32) (width 0.5) (layer "F.Cu") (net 2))
 (segment (start 134.265 49.5) (end 134.265 50.465) (width 0.5) (layer "F.Cu") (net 2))
 (segment (start 140.5 60.5375) (end 142.4 60.5375) (width 0.5) (layer "F.Cu") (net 2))
 (segment (start 142.4 60.5375) (end 149.7175 60.5375) (width 0.5) (layer "F.Cu") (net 2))
 (via (at 142.4 60.5375) (size 0.6) (drill 0.3) (layers "F.Cu" "B.Cu") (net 2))
 (via (at 129.69 63.81) (size 0.8) (drill 0.45) (layers "F.Cu" "B.Cu") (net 2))
 (via (at 136.5375 52.7375) (size 0.6) (drill 0.3) (layers "F.Cu" "B.Cu") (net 2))
 (segment (start 134.46 61.94) (end 135.13 61.27) (width 0.2) (layer "F.Cu") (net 7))
 (segment (start 132.94 63.14) (end 130.14 63.14) (width 0.2) (layer "F.Cu") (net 7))
 (segment (start 138.2 57.860001) (end 137.799999 57.46) (width 0.2) (layer "F.Cu") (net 7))
 (segment (start 135 65.2) (end 132.94 63.14) (width 0.2) (layer "F.Cu") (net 7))
 (segment (start 137.799999 61.27) (end 138.2 60.869999) (width 0.2) (layer "F.Cu") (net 7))
 (segment (start 138.2 60.869999) (end 138.2 57.860001) (width 0.2) (layer "F.Cu") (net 7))
 (segment (start 130.14 63.14) (end 129.9 62.9) (width 0.2) (layer "F.Cu") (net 7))
 (segment (start 129.9 62.9) (end 129.9 62.199448) (width 0.2) (layer "F.Cu") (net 7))
 (segment (start 154.6 65.2) (end 162.2 57.6) (width 0.2) (layer "F.Cu") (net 7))
 (segment (start 140.5 65.2) (end 154.6 65.2) (width 0.2) (layer "F.Cu") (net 7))
 (segment (start 135.13 61.27) (end 136.65 61.27) (width 0.2) (layer "F.Cu") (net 7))
 (segment (start 137.799999 57.46) (end 136.65 57.46) (width 0.2) (layer "F.Cu") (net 7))
 (segment (start 130.159448 61.94) (end 134.46 61.94) (width 0.2) (layer "F.Cu") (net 7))
 (segment (start 162.2 54.095) (end 157.58 49.475) (width 0.2) (layer "F.Cu") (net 7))
 (segment (start 129.9 62.199448) (end 130.159448 61.94) (width 0.2) (layer "F.Cu") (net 7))
 (segment (start 140.5 65.2) (end 135 65.2) (width 0.2) (layer "F.Cu") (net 7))
 (segment (start 136.65 61.27) (end 137.799999 61.27) (width 0.2) (layer "F.Cu") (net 7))
 (segment (start 162.2 57.6) (end 162.2 54.095) (width 0.2) (layer "F.Cu") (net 7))
 (segment (start 131.35 56.19) (end 127.89 56.19) (width 0.2) (layer "F.Cu") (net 8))
 (segment (start 127.5 55.8) (end 127.5 50.7) (width 0.2) (layer "F.Cu") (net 8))
 (segment (start 150.625 47.6) (end 152.5 49.475) (width 0.2) (layer "F.Cu") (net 8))
 (segment (start 127.5 50.7) (end 130.6 47.6) (width 0.2) (layer "F.Cu") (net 8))
 (segment (start 130.6 47.6) (end 150.625 47.6) (width 0.2) (layer "F.Cu") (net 8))
 (segment (start 127.89 56.19) (end 127.5 55.8) (width 0.2) (layer "F.Cu") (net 8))
 (segment (start 127.5 61.3) (end 128.8 60) (width 0.2) (layer "F.Cu") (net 5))
 (segment (start 129.6 60) (end 129.6 58.8) (width 0.2) (layer "F.Cu") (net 5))
 (segment (start 129.67 58.73) (end 131.35 58.73) (width 0.2) (layer "F.Cu") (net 5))
 (segment (start 128.8 60) (end 129.6 60) (width 0.2) (layer "F.Cu") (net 5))
 (segment (start 136.65 60) (end 131.35 60) (width 0.2) (layer "F.Cu") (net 5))
 (segment (start 129.6 58.8) (end 129.67 58.73) (width 0.2) (layer "F.Cu") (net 5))
 (segment (start 129.6 60) (end 131.35 60) (width 0.2) (layer "F.Cu") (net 5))
 (segment (start 141 51) (end 141 49.475) (width 0.2) (layer "F.Cu") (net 6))
 (segment (start 138.8 53.2) (end 141 51) (width 0.2) (layer "F.Cu") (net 6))
 (segment (start 137.799999 62.54) (end 138.8 61.539999) (width 0.2) (layer "F.Cu") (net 6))
 (segment (start 136.65 62.54) (end 137.799999 62.54) (width 0.2) (layer "F.Cu") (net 6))
 (segment (start 138.8 61.539999) (end 138.8 53.2) (width 0.2) (layer "F.Cu") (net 6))
 (segment (start 160.11 55.7) (end 160.12 55.69) (width 0.2) (layer "F.Cu") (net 9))
 (segment (start 142.4 59.4) (end 148.8 59.4) (width 0.2) (layer "F.Cu") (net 9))
 (segment (start 133.93 61.27) (end 131.35 61.27) (width 0.2) (layer "F.Cu") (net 9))
 (segment (start 148.8 59.4) (end 152.5 55.7) (width 0.2) (layer "F.Cu") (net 9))
 (segment (start 134.4 60.8) (end 133.93 61.27) (width 0.2) (layer "F.Cu") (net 9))
 (segment (start 152.5 55.7) (end 160.11 55.7) (width 0.2) (layer "F.Cu") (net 9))
 (via (at 134.4 60.8) (size 0.6) (drill 0.3) (layers "F.Cu" "B.Cu") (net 9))
 (via (at 142.4 59.4) (size 0.6) (drill 0.3) (layers "F.Cu" "B.Cu") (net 9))
 (segment (start 135.8 59.4) (end 142.4 59.4) (width 0.2) (layer "B.Cu") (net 9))
 (segment (start 134.4 60.8) (end 135.8 59.4) (width 0.2) (layer "B.Cu") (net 9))
 (segment (start 140.5 53.8) (end 143.3 53.8) (width 0.2) (layer "F.Cu") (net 4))
 (segment (start 143.3 53.8) (end 146 51.1) (width 0.2) (layer "F.Cu") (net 4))
 (segment (start 146 51.1) (end 146 49.475) (width 0.2) (layer "F.Cu") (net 4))
 (segment (start 139.4 62.209999) (end 139.4 57.3) (width 0.2) (layer "F.Cu") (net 3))
 (segment (start 139.4 57.3) (end 140.5 56.2) (width 0.2) (layer "F.Cu") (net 3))
 (segment (start 133.34 62.54) (end 134.61 63.81) (width 0.2) (layer "F.Cu") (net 3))
 (segment (start 134.61 63.81) (end 136.65 63.81) (width 0.2) (layer "F.Cu") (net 3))
 (segment (start 131.35 62.54) (end 133.34 62.54) (width 0.2) (layer "F.Cu") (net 3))
 (segment (start 137.799999 63.81) (end 139.4 62.209999) (width 0.2) (layer "F.Cu") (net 3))
 (segment (start 136.65 63.81) (end 137.799999 63.81) (width 0.2) (layer "F.Cu") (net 3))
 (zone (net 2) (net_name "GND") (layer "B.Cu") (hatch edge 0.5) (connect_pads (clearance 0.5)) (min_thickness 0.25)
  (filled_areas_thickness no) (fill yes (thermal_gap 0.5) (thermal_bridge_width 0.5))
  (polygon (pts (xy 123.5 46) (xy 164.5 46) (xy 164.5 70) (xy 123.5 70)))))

